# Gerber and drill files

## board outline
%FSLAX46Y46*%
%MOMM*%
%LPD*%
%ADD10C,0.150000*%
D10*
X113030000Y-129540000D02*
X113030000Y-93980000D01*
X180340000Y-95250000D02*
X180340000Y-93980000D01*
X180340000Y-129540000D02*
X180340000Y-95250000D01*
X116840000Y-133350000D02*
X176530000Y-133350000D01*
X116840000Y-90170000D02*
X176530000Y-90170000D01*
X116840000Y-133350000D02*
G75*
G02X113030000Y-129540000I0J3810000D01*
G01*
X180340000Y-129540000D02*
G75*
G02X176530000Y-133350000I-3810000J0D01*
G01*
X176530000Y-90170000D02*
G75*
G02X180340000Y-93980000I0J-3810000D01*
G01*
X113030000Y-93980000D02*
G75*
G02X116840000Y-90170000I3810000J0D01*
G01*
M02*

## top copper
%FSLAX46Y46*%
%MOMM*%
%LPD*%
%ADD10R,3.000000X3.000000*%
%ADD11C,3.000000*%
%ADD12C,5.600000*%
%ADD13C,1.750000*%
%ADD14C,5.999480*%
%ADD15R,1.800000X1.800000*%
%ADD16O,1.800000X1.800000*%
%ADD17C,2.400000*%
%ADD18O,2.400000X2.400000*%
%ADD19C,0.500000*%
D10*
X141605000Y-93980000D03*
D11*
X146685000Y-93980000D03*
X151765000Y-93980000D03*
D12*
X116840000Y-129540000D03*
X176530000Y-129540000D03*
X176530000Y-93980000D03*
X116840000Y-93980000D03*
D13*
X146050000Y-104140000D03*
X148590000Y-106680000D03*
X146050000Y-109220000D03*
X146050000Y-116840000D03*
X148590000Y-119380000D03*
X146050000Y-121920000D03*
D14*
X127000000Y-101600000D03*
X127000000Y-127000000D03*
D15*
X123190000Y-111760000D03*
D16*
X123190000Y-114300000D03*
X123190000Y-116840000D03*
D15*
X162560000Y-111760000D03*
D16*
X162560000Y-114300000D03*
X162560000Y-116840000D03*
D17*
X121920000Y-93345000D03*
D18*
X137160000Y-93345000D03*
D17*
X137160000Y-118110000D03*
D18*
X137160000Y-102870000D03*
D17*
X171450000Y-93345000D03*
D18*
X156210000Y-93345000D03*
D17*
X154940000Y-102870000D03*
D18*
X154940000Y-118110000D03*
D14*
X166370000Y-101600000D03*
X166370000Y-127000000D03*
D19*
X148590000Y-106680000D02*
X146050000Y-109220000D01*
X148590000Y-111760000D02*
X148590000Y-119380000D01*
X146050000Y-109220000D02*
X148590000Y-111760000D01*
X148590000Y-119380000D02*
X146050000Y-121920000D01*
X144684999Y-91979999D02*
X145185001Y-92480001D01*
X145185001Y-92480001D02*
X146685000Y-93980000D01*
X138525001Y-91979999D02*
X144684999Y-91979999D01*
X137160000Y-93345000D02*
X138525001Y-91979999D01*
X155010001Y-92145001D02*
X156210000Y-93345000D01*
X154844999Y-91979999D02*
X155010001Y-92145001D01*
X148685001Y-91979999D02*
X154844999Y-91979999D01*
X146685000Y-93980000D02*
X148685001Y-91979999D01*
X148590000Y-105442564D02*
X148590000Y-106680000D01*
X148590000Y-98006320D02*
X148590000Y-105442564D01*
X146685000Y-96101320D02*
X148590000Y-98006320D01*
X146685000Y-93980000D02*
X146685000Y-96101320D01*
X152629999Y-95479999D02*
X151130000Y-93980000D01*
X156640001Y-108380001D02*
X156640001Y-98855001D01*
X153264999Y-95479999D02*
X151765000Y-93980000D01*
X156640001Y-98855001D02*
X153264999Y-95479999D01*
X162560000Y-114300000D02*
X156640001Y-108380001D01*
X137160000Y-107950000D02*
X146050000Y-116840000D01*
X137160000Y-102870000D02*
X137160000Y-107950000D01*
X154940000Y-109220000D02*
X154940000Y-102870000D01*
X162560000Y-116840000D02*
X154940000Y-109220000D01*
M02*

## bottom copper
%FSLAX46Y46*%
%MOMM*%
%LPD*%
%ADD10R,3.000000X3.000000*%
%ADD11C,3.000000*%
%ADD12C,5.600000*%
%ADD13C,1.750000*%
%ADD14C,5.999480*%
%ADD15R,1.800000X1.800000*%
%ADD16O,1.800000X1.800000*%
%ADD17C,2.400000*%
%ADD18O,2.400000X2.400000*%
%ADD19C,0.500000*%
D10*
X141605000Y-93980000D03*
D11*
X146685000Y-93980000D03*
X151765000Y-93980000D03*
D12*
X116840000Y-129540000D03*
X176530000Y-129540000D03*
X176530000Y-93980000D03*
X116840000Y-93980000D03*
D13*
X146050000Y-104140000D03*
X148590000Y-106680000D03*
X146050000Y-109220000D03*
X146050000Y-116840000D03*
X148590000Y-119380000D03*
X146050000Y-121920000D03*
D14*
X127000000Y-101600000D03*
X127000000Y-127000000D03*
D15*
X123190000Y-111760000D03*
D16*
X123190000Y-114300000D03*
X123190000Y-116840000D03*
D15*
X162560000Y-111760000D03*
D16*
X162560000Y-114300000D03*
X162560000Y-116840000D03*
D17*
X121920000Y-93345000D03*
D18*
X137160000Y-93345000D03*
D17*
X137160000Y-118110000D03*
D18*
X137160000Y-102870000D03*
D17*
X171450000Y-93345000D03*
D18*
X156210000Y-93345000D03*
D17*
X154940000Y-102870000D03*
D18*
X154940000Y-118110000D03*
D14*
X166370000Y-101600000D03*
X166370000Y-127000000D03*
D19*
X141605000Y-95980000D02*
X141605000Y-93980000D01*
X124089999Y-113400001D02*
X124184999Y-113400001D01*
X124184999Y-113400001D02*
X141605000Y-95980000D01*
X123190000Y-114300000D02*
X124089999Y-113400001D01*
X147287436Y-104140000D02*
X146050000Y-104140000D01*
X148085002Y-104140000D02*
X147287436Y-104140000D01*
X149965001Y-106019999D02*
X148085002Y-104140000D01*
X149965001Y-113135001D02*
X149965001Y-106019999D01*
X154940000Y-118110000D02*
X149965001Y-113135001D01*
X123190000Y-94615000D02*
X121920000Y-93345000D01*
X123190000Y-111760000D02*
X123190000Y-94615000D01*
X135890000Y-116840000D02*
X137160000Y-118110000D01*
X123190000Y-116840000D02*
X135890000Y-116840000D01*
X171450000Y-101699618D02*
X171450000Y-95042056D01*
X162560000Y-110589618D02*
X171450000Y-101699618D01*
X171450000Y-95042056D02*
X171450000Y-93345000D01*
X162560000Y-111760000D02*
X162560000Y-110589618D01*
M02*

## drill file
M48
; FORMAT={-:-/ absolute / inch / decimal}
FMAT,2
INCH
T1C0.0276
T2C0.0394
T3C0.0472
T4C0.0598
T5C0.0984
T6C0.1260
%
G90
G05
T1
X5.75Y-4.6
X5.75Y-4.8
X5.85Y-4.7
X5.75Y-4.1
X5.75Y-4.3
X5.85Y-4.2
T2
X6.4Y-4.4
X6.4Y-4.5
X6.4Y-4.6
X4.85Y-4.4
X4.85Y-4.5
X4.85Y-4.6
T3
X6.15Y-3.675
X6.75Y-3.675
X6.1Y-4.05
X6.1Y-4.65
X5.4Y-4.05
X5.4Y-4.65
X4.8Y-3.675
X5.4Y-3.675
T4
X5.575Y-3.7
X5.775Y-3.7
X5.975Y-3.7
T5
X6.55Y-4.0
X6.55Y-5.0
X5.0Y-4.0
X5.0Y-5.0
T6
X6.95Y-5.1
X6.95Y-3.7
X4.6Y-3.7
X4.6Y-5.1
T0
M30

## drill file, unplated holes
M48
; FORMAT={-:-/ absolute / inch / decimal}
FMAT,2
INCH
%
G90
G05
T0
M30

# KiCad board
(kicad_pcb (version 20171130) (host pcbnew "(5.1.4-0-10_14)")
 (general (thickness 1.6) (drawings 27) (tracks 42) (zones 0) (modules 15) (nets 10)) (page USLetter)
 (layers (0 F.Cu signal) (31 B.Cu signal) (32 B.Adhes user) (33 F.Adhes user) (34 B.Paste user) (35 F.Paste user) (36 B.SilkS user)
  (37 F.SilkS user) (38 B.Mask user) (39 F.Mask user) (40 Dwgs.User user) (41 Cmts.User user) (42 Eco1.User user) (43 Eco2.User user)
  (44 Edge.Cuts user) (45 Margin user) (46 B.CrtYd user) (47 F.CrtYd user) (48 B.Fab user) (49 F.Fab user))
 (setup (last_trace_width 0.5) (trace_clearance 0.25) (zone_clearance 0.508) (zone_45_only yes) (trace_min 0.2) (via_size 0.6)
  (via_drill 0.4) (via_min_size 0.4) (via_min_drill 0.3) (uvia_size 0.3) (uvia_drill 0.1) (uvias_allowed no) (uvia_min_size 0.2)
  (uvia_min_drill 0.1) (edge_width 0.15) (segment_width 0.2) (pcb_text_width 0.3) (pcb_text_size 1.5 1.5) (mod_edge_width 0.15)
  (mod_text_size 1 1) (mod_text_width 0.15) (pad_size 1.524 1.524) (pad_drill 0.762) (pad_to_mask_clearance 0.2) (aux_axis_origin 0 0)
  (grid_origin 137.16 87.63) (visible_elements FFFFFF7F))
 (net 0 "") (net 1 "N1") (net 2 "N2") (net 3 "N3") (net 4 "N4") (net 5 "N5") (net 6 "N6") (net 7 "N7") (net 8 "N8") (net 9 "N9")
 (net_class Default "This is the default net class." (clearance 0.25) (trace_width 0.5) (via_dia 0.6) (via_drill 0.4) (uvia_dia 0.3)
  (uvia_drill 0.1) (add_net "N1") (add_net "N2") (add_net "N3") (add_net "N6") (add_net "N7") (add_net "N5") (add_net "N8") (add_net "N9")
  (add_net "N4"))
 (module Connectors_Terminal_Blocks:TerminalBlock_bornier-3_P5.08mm (layer F.Cu) (at 141.605 93.98)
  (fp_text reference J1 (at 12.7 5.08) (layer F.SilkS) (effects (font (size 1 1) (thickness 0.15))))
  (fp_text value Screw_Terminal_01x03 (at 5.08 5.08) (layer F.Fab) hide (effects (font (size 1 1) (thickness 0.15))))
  (pad 1 thru_hole rect (at 0 0) (size 3 3) (drill 1.52) (layers *.Cu *.Mask) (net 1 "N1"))
  (pad 2 thru_hole circle (at 5.08 0) (size 3 3) (drill 1.52) (layers *.Cu *.Mask) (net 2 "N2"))
  (pad 3 thru_hole circle (at 10.16 0) (size 3 3) (drill 1.52) (layers *.Cu *.Mask) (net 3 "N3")))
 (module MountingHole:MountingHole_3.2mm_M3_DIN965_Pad (layer F.Cu) (at 116.84 129.54)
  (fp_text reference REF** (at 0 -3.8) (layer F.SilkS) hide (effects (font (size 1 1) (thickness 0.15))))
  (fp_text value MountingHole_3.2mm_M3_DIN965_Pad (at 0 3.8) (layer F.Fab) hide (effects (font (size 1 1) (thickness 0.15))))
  (pad 1 thru_hole circle (at 0 0) (size 5.6 5.6) (drill 3.2) (layers *.Cu *.Mask)))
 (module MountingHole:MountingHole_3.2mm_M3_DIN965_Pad (layer F.Cu) (at 176.53 129.54)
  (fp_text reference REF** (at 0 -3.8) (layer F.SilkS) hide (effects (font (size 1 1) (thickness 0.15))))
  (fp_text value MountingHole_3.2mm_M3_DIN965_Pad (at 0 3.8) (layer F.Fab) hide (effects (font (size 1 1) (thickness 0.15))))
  (pad 1 thru_hole circle (at 0 0) (size 5.6 5.6) (drill 3.2) (layers *.Cu *.Mask)))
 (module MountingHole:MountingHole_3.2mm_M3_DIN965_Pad (layer F.Cu) (at 176.53 93.98)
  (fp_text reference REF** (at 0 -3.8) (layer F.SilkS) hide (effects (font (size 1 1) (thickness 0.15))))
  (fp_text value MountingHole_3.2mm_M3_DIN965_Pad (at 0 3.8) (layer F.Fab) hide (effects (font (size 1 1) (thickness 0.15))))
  (pad 1 thru_hole circle (at 0 0) (size 5.6 5.6) (drill 3.2) (layers *.Cu *.Mask)))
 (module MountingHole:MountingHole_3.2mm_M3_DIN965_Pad (layer F.Cu) (at 116.84 93.98)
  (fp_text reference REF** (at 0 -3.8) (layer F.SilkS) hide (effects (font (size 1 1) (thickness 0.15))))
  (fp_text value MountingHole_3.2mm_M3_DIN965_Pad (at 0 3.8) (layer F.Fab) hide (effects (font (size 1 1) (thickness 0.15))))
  (pad 1 thru_hole circle (at 0 0) (size 5.6 5.6) (drill 3.2) (layers *.Cu *.Mask)))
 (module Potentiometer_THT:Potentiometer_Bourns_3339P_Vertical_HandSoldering (layer F.Cu) (at 146.05 104.14 180)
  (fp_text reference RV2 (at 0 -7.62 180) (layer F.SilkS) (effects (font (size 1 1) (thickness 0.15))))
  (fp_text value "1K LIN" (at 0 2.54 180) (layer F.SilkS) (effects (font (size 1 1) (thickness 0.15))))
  (pad 1 thru_hole circle (at 0 0 180) (size 1.75 1.75) (drill 0.7) (layers *.Cu *.Mask) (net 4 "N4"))
  (pad 2 thru_hole circle (at -2.54 -2.54 180) (size 1.75 1.75) (drill 0.7) (layers *.Cu *.Mask) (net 2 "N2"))
  (pad 3 thru_hole circle (at 0 -5.08 180) (size 1.75 1.75) (drill 0.7) (layers *.Cu *.Mask) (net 2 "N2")))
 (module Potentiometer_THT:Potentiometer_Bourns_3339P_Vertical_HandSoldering (layer F.Cu) (at 146.05 116.84 180)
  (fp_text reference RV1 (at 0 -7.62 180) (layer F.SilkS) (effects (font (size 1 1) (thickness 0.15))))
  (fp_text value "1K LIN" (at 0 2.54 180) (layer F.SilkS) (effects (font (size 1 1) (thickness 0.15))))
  (pad 1 thru_hole circle (at 0 0 180) (size 1.75 1.75) (drill 0.7) (layers *.Cu *.Mask) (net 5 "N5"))
  (pad 2 thru_hole circle (at -2.54 -2.54 180) (size 1.75 1.75) (drill 0.7) (layers *.Cu *.Mask) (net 2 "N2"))
  (pad 3 thru_hole circle (at 0 -5.08 180) (size 1.75 1.75) (drill 0.7) (layers *.Cu *.Mask) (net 2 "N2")))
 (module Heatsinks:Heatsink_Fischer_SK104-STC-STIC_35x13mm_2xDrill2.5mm (layer F.Cu) (at 127 114.3 90)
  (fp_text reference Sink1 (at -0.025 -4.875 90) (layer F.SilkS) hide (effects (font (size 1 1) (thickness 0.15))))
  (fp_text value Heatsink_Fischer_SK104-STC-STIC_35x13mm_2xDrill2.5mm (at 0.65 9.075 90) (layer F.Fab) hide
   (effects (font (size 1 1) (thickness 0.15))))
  (pad 1 thru_hole circle (at 12.7 0 90) (size 5.99948 5.99948) (drill 2.49936) (layers *.Cu *.Mask))
  (pad 1 thru_hole circle (at -12.7 0 90) (size 5.99948 5.99948) (drill 2.49936) (layers *.Cu *.Mask)))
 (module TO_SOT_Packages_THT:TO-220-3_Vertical (layer F.Cu) (at 123.19 111.76 270)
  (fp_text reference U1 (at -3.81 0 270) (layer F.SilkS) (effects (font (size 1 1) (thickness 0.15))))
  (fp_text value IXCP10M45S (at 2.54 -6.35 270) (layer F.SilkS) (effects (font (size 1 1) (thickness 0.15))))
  (pad 1 thru_hole rect (at 0 0 270) (size 1.8 1.8) (drill 1) (layers *.Cu *.Mask) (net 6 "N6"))
  (pad 2 thru_hole oval (at 2.54 0 270) (size 1.8 1.8) (drill 1) (layers *.Cu *.Mask) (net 1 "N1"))
  (pad 3 thru_hole oval (at 5.08 0 270) (size 1.8 1.8) (drill 1) (layers *.Cu *.Mask) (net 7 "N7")))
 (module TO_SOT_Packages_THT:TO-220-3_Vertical (layer F.Cu) (at 162.56 111.76 270)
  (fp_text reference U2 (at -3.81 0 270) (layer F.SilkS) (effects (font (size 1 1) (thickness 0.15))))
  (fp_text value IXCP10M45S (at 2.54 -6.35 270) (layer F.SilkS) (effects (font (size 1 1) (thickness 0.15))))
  (pad 1 thru_hole rect (at 0 0 270) (size 1.8 1.8) (drill 1) (layers *.Cu *.Mask) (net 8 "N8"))
  (pad 2 thru_hole oval (at 2.54 0 270) (size 1.8 1.8) (drill 1) (layers *.Cu *.Mask) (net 3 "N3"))
  (pad 3 thru_hole oval (at 5.08 0 270) (size 1.8 1.8) (drill 1) (layers *.Cu *.Mask) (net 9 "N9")))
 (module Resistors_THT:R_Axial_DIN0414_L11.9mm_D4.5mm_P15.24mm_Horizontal (layer F.Cu) (at 121.92 93.345)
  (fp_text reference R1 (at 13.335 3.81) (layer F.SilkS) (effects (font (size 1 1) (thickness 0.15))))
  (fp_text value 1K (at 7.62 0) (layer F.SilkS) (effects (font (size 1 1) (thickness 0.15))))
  (pad 1 thru_hole circle (at 0 0) (size 2.4 2.4) (drill 1.2) (layers *.Cu *.Mask) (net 6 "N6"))
  (pad 2 thru_hole oval (at 15.24 0) (size 2.4 2.4) (drill 1.2) (layers *.Cu *.Mask) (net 2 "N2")))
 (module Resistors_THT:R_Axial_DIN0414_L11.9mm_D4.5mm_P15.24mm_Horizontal (layer F.Cu) (at 137.16 118.11 90)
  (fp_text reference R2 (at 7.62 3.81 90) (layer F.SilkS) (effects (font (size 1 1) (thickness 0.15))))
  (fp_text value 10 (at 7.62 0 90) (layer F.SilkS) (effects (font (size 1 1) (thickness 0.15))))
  (pad 1 thru_hole circle (at 0 0 90) (size 2.4 2.4) (drill 1.2) (layers *.Cu *.Mask) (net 7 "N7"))
  (pad 2 thru_hole oval (at 15.24 0 90) (size 2.4 2.4) (drill 1.2) (layers *.Cu *.Mask) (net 5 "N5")))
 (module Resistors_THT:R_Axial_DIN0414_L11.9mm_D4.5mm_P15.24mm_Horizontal (layer F.Cu) (at 171.45 93.345 180)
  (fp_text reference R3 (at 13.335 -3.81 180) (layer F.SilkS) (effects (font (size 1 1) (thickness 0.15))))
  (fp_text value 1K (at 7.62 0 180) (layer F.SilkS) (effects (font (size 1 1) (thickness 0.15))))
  (pad 1 thru_hole circle (at 0 0 180) (size 2.4 2.4) (drill 1.2) (layers *.Cu *.Mask) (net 8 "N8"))
  (pad 2 thru_hole oval (at 15.24 0 180) (size 2.4 2.4) (drill 1.2) (layers *.Cu *.Mask) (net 2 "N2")))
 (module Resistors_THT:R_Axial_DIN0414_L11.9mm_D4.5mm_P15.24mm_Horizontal (layer F.Cu) (at 154.94 102.87 270)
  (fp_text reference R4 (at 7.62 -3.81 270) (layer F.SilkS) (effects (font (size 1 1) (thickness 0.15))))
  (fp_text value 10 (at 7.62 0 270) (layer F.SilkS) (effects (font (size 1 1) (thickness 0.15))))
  (pad 1 thru_hole circle (at 0 0 270) (size 2.4 2.4) (drill 1.2) (layers *.Cu *.Mask) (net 9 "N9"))
  (pad 2 thru_hole oval (at 15.24 0 270) (size 2.4 2.4) (drill 1.2) (layers *.Cu *.Mask) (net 4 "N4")))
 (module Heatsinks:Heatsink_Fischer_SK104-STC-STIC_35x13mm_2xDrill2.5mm (layer F.Cu) (at 166.37 114.3 90)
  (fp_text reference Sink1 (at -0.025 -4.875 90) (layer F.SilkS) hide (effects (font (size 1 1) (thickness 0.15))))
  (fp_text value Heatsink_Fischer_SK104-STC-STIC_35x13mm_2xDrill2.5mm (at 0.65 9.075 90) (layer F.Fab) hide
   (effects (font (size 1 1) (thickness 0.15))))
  (pad 1 thru_hole circle (at 12.7 0 90) (size 5.99948 5.99948) (drill 2.49936) (layers *.Cu *.Mask))
  (pad 1 thru_hole circle (at -12.7 0 90) (size 5.99948 5.99948) (drill 2.49936) (layers *.Cu *.Mask)))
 (gr_line (start 113.03 129.54) (end 113.03 93.98) (layer Edge.Cuts) (width 0.15))
 (gr_line (start 180.34 95.25) (end 180.34 93.98) (layer Edge.Cuts) (width 0.15))
 (gr_line (start 180.34 129.54) (end 180.34 95.25) (layer Edge.Cuts) (width 0.15))
 (gr_line (start 116.84 133.35) (end 176.53 133.35) (layer Edge.Cuts) (width 0.15))
 (gr_line (start 116.84 90.17) (end 176.53 90.17) (layer Edge.Cuts) (width 0.15))
 (gr_arc (start 116.84 129.54) (end 113.03 129.54) (angle -90) (layer Edge.Cuts) (width 0.15))
 (gr_arc (start 176.53 129.54) (end 176.53 133.35) (angle -90) (layer Edge.Cuts) (width 0.15))
 (gr_arc (start 176.53 93.98) (end 180.34 93.98) (angle -90) (layer Edge.Cuts) (width 0.15))
 (gr_arc (start 116.84 93.98) (end 116.84 90.17) (angle -90) (layer Edge.Cuts) (width 0.15))
 (segment (start 141.605 95.98) (end 141.605 93.98) (width 0.5) (layer B.Cu) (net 1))
 (segment (start 124.089999 113.400001) (end 124.184999 113.400001) (width 0.5) (layer B.Cu) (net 1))
 (segment (start 124.184999 113.400001) (end 141.605 95.98) (width 0.5) (layer B.Cu) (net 1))
 (segment (start 123.19 114.3) (end 124.089999 113.400001) (width 0.5) (layer B.Cu) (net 1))
 (segment (start 148.59 106.68) (end 146.05 109.22) (width 0.5) (layer F.Cu) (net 2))
 (segment (start 148.59 111.76) (end 148.59 119.38) (width 0.5) (layer F.Cu) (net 2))
 (segment (start 146.05 109.22) (end 148.59 111.76) (width 0.5) (layer F.Cu) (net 2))
 (segment (start 148.59 119.38) (end 146.05 121.92) (width 0.5) (layer F.Cu) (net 2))
 (segment (start 144.684999 91.979999) (end 145.185001 92.480001) (width 0.5) (layer F.Cu) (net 2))
 (segment (start 145.185001 92.480001) (end 146.685 93.98) (width 0.5) (layer F.Cu) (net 2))
 (segment (start 138.525001 91.979999) (end 144.684999 91.979999) (width 0.5) (layer F.Cu) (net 2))
 (segment (start 137.16 93.345) (end 138.525001 91.979999) (width 0.5) (layer F.Cu) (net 2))
 (segment (start 155.010001 92.145001) (end 156.21 93.345) (width 0.5) (layer F.Cu) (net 2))
 (segment (start 154.844999 91.979999) (end 155.010001 92.145001) (width 0.5) (layer F.Cu) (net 2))
 (segment (start 148.685001 91.979999) (end 154.844999 91.979999) (width 0.5) (layer F.Cu) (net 2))
 (segment (start 146.685 93.98) (end 148.685001 91.979999) (width 0.5) (layer F.Cu) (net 2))
 (segment (start 148.59 105.442564) (end 148.59 106.68) (width 0.5) (layer F.Cu) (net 2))
 (segment (start 148.59 98.00632) (end 148.59 105.442564) (width 0.5) (layer F.Cu) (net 2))
 (segment (start 146.685 96.10132) (end 148.59 98.00632) (width 0.5) (layer F.Cu) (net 2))
 (segment (start 146.685 93.98) (end 146.685 96.10132) (width 0.5) (layer F.Cu) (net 2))
 (segment (start 152.629999 95.479999) (end 151.13 93.98) (width 0.5) (layer F.Cu) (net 3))
 (segment (start 156.640001 108.380001) (end 156.640001 98.855001) (width 0.5) (layer F.Cu) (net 3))
 (segment (start 153.264999 95.479999) (end 151.765 93.98) (width 0.5) (layer F.Cu) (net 3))
 (segment (start 156.640001 98.855001) (end 153.264999 95.479999) (width 0.5) (layer F.Cu) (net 3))
 (segment (start 162.56 114.3) (end 156.640001 108.380001) (width 0.5) (layer F.Cu) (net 3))
 (segment (start 137.16 107.95) (end 146.05 116.84) (width 0.5) (layer F.Cu) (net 5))
 (segment (start 137.16 102.87) (end 137.16 107.95) (width 0.5) (layer F.Cu) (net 5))
 (segment (start 147.287436 104.14) (end 146.05 104.14) (width 0.5) (layer B.Cu) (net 4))
 (segment (start 148.085002 104.14) (end 147.287436 104.14) (width 0.5) (layer B.Cu) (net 4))
 (segment (start 149.965001 106.019999) (end 148.085002 104.14) (width 0.5) (layer B.Cu) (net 4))
 (segment (start 149.965001 113.135001) (end 149.965001 106.019999) (width 0.5) (layer B.Cu) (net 4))
 (segment (start 154.94 118.11) (end 149.965001 113.135001) (width 0.5) (layer B.Cu) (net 4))
 (segment (start 123.19 94.615) (end 121.92 93.345) (width 0.5) (layer B.Cu) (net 6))
 (segment (start 123.19 111.76) (end 123.19 94.615) (width 0.5) (layer B.Cu) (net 6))
 (segment (start 135.89 116.84) (end 137.16 118.11) (width 0.5) (layer B.Cu) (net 7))
 (segment (start 123.19 116.84) (end 135.89 116.84) (width 0.5) (layer B.Cu) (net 7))
 (segment (start 171.45 101.699618) (end 171.45 95.042056) (width 0.5) (layer B.Cu) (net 8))
 (segment (start 162.56 110.589618) (end 171.45 101.699618) (width 0.5) (layer B.Cu) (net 8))
 (segment (start 171.45 95.042056) (end 171.45 93.345) (width 0.5) (layer B.Cu) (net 8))
 (segment (start 162.56 111.76) (end 162.56 110.589618) (width 0.5) (layer B.Cu) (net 8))
 (segment (start 154.94 109.22) (end 154.94 102.87) (width 0.5) (layer F.Cu) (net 9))
 (segment (start 162.56 116.84) (end 154.94 109.22) (width 0.5) (layer F.Cu) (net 9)))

